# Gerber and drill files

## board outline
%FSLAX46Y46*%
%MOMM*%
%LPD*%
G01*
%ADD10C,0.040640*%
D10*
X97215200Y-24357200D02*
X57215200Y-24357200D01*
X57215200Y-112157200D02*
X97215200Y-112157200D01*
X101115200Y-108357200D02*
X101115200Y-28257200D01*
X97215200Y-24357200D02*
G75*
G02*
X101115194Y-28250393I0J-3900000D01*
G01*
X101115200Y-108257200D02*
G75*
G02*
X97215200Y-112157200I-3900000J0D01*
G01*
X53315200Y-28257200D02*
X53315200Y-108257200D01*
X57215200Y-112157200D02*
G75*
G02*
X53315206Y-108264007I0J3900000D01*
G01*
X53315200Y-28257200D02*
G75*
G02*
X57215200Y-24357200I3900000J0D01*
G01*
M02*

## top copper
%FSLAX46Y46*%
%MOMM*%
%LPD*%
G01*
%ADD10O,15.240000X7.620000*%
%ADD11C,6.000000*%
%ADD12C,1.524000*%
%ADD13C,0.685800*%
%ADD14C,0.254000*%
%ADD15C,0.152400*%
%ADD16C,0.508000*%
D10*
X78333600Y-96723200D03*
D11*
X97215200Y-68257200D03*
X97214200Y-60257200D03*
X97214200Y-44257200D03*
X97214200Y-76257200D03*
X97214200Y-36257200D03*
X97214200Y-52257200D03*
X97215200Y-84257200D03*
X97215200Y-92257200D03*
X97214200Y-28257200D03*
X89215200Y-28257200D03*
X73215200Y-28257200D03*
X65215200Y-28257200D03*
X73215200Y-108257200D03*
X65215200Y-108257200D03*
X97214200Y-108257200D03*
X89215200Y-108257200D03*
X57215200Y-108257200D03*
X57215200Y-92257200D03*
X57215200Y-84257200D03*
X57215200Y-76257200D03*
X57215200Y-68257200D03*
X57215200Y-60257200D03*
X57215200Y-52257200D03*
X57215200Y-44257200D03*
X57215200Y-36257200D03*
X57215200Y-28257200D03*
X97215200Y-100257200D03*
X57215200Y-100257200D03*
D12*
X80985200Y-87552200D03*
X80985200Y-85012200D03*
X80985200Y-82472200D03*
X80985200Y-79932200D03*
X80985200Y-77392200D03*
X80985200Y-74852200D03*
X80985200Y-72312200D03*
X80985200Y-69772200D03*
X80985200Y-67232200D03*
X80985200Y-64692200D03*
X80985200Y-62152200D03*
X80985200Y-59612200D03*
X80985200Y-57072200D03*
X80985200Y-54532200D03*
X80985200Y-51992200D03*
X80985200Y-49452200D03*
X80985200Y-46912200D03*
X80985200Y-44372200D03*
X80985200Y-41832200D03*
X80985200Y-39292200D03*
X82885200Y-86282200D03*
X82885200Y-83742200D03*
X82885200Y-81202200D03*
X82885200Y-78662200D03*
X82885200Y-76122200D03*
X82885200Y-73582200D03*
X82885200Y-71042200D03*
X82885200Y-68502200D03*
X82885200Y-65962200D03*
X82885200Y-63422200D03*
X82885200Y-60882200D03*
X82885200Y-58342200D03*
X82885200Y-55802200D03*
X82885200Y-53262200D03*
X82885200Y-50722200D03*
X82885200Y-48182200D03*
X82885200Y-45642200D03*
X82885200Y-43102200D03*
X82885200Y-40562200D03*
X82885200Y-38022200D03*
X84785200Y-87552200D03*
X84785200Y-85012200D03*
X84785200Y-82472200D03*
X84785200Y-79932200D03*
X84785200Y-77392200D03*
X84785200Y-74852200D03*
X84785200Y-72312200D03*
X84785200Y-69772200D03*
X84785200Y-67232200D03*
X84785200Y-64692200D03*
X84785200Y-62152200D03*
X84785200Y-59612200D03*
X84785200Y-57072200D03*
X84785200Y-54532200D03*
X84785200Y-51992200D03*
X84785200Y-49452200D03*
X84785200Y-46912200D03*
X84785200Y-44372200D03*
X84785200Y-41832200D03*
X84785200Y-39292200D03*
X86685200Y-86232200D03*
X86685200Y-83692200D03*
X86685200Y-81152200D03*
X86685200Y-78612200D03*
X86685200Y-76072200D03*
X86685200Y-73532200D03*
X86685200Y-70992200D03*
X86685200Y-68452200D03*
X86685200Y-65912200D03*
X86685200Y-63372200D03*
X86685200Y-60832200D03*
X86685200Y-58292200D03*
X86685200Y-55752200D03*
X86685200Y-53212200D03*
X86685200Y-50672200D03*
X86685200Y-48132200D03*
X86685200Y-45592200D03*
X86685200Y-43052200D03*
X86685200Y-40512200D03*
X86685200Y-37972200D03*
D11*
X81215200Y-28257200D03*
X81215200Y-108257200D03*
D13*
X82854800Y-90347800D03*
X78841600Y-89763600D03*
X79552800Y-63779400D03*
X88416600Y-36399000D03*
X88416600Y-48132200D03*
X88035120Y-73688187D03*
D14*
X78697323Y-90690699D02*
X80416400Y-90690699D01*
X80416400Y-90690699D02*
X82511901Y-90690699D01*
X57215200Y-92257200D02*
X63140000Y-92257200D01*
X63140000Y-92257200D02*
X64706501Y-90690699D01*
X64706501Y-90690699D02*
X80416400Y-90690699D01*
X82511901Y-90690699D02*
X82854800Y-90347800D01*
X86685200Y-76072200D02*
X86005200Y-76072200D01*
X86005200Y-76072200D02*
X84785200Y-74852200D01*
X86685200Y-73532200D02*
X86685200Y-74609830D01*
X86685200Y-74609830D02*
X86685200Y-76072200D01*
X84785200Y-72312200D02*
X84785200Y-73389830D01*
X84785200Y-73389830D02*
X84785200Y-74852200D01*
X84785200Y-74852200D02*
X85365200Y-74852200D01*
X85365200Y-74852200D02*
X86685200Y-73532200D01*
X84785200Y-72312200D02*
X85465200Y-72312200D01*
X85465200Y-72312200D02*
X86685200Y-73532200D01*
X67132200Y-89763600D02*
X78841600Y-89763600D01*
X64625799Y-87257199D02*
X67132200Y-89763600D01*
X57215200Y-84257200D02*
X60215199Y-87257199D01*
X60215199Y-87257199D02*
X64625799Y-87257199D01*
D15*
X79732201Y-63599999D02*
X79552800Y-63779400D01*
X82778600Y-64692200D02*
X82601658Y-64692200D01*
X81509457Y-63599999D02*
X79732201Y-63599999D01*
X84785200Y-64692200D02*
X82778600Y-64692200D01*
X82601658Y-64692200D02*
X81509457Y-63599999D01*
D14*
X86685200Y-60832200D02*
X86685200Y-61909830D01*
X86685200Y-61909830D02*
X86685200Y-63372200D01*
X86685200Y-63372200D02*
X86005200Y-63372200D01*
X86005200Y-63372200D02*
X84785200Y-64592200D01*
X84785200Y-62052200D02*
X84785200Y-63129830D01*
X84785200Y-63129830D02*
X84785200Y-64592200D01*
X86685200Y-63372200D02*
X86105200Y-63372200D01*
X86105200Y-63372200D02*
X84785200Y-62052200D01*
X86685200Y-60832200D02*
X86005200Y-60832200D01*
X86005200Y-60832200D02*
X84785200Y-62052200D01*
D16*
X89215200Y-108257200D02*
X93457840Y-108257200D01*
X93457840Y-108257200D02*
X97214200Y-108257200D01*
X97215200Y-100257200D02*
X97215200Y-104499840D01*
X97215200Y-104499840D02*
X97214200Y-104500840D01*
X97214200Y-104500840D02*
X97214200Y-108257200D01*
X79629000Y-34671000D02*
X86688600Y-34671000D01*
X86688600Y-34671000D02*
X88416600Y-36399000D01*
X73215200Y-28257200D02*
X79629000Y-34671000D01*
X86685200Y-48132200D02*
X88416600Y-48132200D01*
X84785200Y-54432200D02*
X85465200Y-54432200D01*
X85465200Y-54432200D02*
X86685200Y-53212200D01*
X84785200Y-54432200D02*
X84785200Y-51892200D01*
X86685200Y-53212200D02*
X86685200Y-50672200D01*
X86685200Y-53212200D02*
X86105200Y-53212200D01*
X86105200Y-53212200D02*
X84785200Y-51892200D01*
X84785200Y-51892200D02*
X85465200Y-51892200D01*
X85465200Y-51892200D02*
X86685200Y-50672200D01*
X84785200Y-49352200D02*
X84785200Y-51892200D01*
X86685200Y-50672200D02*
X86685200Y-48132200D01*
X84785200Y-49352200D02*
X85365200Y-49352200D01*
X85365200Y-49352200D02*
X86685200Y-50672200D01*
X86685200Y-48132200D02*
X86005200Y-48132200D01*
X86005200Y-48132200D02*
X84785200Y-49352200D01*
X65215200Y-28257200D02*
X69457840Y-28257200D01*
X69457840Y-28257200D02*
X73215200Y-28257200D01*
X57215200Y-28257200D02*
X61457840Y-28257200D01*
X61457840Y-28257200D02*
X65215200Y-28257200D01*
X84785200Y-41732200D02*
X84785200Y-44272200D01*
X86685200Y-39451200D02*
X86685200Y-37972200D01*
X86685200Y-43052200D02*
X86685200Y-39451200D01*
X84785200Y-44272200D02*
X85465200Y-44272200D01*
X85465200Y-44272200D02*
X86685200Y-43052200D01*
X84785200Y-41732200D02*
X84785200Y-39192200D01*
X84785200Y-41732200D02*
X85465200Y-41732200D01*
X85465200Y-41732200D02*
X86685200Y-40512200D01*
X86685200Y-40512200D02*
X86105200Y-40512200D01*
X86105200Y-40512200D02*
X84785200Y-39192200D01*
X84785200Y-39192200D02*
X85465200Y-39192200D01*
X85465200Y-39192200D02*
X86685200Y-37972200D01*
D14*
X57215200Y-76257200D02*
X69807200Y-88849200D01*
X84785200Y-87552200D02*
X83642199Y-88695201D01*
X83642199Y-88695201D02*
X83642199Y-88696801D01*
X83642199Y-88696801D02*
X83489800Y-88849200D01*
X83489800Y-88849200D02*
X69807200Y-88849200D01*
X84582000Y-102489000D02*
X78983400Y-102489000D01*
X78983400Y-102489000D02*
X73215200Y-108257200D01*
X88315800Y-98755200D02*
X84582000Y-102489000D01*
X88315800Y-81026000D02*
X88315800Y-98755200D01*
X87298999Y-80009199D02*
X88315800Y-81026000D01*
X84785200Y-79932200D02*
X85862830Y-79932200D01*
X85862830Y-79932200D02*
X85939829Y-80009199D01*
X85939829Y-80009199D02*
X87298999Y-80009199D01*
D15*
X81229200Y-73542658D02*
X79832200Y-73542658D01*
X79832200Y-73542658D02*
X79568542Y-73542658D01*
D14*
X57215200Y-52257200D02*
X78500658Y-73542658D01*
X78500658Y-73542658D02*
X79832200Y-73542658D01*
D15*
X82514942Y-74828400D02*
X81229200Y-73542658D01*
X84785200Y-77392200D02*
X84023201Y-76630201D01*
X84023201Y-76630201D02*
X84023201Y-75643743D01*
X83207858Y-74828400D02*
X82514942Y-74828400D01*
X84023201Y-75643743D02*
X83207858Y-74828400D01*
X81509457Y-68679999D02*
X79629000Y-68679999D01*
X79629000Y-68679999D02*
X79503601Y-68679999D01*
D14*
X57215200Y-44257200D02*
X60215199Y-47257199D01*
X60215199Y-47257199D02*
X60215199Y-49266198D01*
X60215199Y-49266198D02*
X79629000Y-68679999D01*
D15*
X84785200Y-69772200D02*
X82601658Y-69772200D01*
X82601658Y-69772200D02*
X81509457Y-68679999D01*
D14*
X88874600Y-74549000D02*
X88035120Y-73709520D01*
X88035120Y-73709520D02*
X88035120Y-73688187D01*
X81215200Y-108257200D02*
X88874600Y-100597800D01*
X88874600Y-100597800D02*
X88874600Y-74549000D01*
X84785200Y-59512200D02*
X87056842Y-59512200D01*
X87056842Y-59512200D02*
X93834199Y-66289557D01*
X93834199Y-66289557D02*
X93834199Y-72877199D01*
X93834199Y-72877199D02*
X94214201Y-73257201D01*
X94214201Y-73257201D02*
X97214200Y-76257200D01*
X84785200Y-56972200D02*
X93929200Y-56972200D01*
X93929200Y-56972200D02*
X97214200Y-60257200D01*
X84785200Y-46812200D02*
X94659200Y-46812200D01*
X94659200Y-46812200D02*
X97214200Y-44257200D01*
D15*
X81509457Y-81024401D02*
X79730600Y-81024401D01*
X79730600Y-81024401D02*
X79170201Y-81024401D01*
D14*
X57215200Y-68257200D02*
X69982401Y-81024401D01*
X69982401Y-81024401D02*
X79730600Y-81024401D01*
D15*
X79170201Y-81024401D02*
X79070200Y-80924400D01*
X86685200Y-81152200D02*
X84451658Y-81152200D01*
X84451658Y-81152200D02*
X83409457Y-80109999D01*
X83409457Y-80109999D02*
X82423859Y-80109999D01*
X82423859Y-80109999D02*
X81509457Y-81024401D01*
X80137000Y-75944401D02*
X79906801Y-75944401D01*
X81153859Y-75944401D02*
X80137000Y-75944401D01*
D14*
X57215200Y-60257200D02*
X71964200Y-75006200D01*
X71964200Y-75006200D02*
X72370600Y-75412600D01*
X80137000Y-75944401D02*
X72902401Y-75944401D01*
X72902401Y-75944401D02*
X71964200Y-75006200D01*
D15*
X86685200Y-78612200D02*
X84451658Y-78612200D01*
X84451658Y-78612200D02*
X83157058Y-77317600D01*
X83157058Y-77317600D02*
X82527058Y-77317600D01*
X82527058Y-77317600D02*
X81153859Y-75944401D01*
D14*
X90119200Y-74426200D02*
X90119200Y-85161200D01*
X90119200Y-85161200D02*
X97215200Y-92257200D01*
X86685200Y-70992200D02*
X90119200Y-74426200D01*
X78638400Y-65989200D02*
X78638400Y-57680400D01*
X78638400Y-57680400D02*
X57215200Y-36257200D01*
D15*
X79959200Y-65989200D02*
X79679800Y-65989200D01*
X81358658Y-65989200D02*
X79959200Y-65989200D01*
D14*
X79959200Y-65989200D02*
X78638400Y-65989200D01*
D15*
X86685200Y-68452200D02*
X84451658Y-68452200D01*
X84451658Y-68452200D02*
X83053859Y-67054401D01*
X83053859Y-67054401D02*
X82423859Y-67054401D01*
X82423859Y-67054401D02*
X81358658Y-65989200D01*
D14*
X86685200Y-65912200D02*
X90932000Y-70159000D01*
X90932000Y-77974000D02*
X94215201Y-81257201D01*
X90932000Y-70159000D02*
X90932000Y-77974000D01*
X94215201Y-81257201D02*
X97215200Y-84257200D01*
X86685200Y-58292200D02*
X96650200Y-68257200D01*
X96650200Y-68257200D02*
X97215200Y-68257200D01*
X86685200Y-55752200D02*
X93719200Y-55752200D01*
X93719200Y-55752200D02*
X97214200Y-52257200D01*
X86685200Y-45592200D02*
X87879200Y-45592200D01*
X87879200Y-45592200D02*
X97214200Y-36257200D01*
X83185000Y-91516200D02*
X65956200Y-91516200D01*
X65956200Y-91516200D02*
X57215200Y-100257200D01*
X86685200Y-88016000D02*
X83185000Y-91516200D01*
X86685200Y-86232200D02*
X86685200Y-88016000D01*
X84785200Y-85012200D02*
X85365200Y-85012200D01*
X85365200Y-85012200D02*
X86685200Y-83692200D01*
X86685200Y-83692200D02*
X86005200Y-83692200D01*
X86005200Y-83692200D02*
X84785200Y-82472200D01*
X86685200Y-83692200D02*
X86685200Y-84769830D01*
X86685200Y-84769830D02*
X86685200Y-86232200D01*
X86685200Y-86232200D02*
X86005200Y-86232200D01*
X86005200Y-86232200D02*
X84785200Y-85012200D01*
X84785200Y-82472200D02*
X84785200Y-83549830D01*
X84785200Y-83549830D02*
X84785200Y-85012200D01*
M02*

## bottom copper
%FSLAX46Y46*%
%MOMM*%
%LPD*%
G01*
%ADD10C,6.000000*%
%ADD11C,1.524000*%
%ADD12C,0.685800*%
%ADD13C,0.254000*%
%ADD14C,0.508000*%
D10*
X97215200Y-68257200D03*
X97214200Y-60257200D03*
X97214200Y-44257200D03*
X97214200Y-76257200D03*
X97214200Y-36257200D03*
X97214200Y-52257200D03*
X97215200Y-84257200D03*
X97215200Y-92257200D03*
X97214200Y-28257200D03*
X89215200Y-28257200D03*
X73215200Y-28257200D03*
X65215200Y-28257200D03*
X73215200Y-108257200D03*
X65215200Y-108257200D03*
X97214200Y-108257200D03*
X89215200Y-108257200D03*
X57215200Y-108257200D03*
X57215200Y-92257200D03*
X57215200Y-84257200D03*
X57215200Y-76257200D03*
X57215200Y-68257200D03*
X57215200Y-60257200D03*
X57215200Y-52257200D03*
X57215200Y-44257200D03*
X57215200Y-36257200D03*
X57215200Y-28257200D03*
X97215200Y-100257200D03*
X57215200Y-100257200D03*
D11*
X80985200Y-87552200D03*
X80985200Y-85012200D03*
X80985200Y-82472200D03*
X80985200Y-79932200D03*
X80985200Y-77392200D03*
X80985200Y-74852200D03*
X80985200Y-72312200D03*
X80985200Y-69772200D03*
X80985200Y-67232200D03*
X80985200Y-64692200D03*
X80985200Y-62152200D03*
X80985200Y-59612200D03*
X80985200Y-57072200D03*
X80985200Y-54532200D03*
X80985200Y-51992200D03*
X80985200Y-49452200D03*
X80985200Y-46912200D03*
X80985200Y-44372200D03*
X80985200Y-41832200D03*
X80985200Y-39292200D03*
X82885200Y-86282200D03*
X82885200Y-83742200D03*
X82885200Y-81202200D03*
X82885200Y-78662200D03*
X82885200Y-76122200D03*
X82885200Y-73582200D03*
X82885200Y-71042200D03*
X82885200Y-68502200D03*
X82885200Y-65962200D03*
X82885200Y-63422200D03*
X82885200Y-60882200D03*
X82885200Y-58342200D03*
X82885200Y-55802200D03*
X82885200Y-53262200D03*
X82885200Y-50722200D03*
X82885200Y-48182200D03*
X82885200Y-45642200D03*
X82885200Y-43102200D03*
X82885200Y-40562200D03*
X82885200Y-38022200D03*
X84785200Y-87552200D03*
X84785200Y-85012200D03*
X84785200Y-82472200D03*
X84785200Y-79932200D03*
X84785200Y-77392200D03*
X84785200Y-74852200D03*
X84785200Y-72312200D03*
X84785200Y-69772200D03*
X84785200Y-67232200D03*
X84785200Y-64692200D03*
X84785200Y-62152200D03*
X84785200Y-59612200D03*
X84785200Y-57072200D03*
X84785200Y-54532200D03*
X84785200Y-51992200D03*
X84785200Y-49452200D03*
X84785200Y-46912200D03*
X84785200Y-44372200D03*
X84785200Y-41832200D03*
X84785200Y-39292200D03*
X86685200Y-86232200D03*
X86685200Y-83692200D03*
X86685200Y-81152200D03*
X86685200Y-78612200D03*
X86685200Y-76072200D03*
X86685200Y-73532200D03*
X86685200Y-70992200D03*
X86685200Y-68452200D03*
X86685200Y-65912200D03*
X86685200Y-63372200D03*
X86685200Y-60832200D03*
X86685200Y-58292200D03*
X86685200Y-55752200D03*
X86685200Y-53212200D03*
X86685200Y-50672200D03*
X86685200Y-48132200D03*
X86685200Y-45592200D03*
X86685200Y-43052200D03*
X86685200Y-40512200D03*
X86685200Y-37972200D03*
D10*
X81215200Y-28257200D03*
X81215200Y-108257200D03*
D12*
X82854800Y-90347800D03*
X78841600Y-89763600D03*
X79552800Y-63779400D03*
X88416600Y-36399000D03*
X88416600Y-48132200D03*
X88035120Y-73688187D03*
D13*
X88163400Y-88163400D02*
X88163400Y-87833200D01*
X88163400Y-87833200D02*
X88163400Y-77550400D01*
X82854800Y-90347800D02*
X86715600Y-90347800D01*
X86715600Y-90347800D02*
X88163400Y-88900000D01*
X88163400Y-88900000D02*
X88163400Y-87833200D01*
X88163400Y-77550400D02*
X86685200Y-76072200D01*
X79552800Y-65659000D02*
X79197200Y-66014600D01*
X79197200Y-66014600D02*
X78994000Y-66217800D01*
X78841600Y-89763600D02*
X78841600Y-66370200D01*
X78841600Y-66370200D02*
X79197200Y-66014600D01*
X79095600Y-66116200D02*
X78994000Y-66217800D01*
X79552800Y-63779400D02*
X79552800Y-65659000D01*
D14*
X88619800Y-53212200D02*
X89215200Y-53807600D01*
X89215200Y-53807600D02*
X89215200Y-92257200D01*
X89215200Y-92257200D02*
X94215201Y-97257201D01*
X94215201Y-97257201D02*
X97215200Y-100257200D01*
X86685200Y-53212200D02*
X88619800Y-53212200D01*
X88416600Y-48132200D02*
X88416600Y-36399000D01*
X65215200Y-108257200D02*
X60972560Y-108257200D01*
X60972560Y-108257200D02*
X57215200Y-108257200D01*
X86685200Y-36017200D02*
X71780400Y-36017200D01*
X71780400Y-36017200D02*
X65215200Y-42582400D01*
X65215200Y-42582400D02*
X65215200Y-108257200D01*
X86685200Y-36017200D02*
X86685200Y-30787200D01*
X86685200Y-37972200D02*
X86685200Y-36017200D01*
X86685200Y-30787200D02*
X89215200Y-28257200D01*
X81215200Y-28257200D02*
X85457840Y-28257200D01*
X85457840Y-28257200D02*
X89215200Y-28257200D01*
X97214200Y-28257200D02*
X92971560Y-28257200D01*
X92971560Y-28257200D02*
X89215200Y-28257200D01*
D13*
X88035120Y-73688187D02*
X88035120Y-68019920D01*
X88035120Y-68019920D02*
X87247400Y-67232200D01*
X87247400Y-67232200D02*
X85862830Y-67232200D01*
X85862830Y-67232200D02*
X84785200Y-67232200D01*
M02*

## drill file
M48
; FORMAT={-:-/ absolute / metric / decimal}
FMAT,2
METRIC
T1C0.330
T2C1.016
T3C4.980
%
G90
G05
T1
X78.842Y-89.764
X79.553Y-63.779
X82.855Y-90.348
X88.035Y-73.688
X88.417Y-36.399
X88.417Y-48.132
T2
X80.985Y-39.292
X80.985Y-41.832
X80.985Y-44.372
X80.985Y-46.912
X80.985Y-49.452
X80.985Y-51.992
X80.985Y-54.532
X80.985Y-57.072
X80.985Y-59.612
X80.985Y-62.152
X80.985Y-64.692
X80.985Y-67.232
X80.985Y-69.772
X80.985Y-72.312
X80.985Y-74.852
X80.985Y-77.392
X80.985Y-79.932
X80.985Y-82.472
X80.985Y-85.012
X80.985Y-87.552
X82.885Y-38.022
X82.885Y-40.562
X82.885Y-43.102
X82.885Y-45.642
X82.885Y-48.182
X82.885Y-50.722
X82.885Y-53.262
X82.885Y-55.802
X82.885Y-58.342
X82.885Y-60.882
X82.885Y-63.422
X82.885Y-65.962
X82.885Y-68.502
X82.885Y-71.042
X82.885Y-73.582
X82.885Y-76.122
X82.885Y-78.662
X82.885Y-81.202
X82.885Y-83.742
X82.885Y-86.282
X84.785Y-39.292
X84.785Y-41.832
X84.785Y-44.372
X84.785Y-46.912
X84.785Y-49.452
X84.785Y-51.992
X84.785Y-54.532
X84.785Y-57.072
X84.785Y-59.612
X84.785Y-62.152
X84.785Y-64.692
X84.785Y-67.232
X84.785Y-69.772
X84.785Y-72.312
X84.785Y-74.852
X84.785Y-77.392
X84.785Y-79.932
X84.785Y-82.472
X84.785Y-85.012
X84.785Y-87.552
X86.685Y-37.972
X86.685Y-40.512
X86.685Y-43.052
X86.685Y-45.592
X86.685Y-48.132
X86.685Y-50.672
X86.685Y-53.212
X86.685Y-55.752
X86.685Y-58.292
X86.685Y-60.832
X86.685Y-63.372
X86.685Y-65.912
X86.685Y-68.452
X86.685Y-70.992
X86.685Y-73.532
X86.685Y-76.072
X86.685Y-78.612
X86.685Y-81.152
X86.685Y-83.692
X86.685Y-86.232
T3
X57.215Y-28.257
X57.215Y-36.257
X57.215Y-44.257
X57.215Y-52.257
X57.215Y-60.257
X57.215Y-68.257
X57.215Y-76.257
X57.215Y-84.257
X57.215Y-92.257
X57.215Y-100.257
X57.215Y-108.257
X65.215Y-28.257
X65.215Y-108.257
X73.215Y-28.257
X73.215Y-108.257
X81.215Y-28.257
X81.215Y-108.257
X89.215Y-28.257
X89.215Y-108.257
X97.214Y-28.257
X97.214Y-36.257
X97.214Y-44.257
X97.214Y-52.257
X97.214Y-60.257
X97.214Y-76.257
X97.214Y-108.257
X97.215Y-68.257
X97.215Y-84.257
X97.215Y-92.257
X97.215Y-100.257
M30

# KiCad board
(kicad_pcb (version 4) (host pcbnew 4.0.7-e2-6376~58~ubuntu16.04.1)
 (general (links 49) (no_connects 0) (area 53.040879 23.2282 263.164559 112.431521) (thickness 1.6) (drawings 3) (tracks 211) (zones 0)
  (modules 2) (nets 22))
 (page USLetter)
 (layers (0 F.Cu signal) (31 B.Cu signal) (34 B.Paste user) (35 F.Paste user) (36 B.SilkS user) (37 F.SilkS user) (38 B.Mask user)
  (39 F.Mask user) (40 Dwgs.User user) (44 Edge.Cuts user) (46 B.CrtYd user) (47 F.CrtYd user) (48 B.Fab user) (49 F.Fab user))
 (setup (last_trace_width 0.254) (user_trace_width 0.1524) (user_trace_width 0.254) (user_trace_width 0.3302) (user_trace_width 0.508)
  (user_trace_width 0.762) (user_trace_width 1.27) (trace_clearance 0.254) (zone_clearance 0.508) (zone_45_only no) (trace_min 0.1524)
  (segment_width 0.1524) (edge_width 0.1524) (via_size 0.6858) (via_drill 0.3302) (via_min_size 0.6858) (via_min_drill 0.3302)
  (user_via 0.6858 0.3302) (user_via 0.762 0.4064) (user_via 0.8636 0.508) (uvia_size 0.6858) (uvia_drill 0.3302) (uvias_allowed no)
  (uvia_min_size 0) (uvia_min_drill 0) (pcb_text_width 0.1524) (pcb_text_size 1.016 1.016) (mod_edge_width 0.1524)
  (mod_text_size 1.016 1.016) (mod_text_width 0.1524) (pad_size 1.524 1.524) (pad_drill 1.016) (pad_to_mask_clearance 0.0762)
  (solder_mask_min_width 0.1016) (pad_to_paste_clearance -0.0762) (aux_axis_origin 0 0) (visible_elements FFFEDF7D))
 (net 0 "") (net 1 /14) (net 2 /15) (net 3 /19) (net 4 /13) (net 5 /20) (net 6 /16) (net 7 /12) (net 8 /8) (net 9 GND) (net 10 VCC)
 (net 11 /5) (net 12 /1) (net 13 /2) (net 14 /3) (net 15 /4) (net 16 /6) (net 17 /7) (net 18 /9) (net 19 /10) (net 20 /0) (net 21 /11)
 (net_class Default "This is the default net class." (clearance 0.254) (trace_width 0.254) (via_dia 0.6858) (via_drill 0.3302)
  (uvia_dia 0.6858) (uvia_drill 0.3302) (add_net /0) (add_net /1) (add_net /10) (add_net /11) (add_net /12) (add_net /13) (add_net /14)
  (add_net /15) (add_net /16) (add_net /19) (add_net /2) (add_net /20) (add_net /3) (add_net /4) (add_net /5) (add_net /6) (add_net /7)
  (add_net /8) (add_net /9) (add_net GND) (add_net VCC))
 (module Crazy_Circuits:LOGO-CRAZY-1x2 (layer F.Cu) (at 78.3336 100.6602)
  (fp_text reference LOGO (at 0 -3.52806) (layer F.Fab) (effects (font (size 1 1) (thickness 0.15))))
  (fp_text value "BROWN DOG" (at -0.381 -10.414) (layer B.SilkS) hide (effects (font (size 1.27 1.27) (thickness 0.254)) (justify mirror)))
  (pad BG smd oval (at 0 -3.937) (size 15.24 7.62) (layers F.Cu)))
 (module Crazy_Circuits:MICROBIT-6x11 (layer F.Cu) (at 57.2152 28.2572)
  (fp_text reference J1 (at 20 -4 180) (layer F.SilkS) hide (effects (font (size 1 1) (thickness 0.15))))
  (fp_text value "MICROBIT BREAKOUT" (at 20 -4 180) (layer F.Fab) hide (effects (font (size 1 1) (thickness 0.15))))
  (fp_line (start 40 -3.9) (end 0 -3.9) (layer Edge.Cuts) (width 0.04064))
  (fp_line (start 0 83.9) (end 40 83.9) (layer Edge.Cuts) (width 0.04064))
  (fp_line (start 43.9 80.1) (end 43.9 0) (layer Edge.Cuts) (width 0.04064))
  (fp_arc (start 40 0) (end 40 -3.9) (angle 89.9) (layer Edge.Cuts) (width 0.04064))
  (fp_arc (start 40 80) (end 43.9 80) (angle 90) (layer Edge.Cuts) (width 0.04064))
  (fp_line (start -3.9 0) (end -3.9 80) (layer Edge.Cuts) (width 0.04064))
  (fp_arc (start 0 80) (end 0 83.9) (angle 89.9) (layer Edge.Cuts) (width 0.04064))
  (fp_arc (start 0 0) (end -3.9 0) (angle 90) (layer Edge.Cuts) (width 0.04064))
  (pad 14 thru_hole circle (at 40 40 270) (size 6 6) (drill 4.98) (layers *.Cu *.Mask) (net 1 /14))
  (pad 15 thru_hole circle (at 39.999 32 270) (size 6 6) (drill 4.98) (layers *.Cu *.Mask) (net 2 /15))
  (pad 19 thru_hole circle (at 39.999 16 270) (size 6 6) (drill 4.98) (layers *.Cu *.Mask) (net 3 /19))
  (pad 13 thru_hole circle (at 39.999 48 270) (size 6 6) (drill 4.98) (layers *.Cu *.Mask) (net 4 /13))
  (pad 20 thru_hole circle (at 39.999 8 270) (size 6 6) (drill 4.98) (layers *.Cu *.Mask) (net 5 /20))
  (pad 16 thru_hole circle (at 39.999 24 270) (size 6 6) (drill 4.98) (layers *.Cu *.Mask) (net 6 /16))
  (pad 12 thru_hole circle (at 40 56 270) (size 6 6) (drill 4.98) (layers *.Cu *.Mask) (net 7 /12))
  (pad 8 thru_hole circle (at 40 64 270) (size 6 6) (drill 4.98) (layers *.Cu *.Mask) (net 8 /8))
  (pad GND thru_hole circle (at 39.999 0 270) (size 6 6) (drill 4.98) (layers *.Cu *.Mask) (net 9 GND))
  (pad GND thru_hole circle (at 32 0 270) (size 6 6) (drill 4.98) (layers *.Cu *.Mask) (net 9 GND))
  (pad 3V thru_hole circle (at 16 0 270) (size 6 6) (drill 4.98) (layers *.Cu *.Mask) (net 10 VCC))
  (pad 3V thru_hole circle (at 8 0 270) (size 6 6) (drill 4.98) (layers *.Cu *.Mask) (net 10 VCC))
  (pad 5 thru_hole circle (at 16 80 270) (size 6 6) (drill 4.98) (layers *.Cu *.Mask) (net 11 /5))
  (pad GND thru_hole circle (at 8 80 270) (size 6 6) (drill 4.98) (layers *.Cu *.Mask) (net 9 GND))
  (pad 3V thru_hole circle (at 39.999 80 270) (size 6 6) (drill 4.98) (layers *.Cu *.Mask) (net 10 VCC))
  (pad 3V thru_hole circle (at 32 80 270) (size 6 6) (drill 4.98) (layers *.Cu *.Mask) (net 10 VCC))
  (pad GND thru_hole circle (at 0 80 270) (size 6 6) (drill 4.98) (layers *.Cu *.Mask) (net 9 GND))
  (pad 1 thru_hole circle (at 0 64 270) (size 6 6) (drill 4.98) (layers *.Cu *.Mask) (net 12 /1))
  (pad 2 thru_hole circle (at 0 56 270) (size 6 6) (drill 4.98) (layers *.Cu *.Mask) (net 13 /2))
  (pad 3 thru_hole circle (at 0 48 270) (size 6 6) (drill 4.98) (layers *.Cu *.Mask) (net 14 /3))
  (pad 4 thru_hole circle (at 0 40 270) (size 6 6) (drill 4.98) (layers *.Cu *.Mask) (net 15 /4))
  (pad 6 thru_hole circle (at 0 32 270) (size 6 6) (drill 4.98) (layers *.Cu *.Mask) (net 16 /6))
  (pad 7 thru_hole circle (at 0 24 270) (size 6 6) (drill 4.98) (layers *.Cu *.Mask) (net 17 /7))
  (pad 9 thru_hole circle (at 0 16 270) (size 6 6) (drill 4.98) (layers *.Cu *.Mask) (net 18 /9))
  (pad 10 thru_hole circle (at 0 8 270) (size 6 6) (drill 4.98) (layers *.Cu *.Mask) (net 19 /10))
  (pad 3V thru_hole circle (at 0 0 270) (size 6 6) (drill 4.98) (layers *.Cu *.Mask) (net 10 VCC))
  (pad 3V thru_hole circle (at 40 72 270) (size 6 6) (drill 4.98) (layers *.Cu *.Mask) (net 10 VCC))
  (pad 0 thru_hole circle (at 0 72 270) (size 6 6) (drill 4.98) (layers *.Cu *.Mask) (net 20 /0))
  (pad NC thru_hole circle (at 23.77 59.295 90) (size 1.524 1.524) (drill 1.016) (layers *.Cu *.Mask F.SilkS))
  (pad NC thru_hole circle (at 23.77 56.755 90) (size 1.524 1.524) (drill 1.016) (layers *.Cu *.Mask F.SilkS))
  (pad NC thru_hole circle (at 23.77 54.215 90) (size 1.524 1.524) (drill 1.016) (layers *.Cu *.Mask F.SilkS))
  (pad NC thru_hole circle (at 23.77 51.675 90) (size 1.524 1.524) (drill 1.016) (layers *.Cu *.Mask F.SilkS))
  (pad NC thru_hole circle (at 23.77 49.135 90) (size 1.524 1.524) (drill 1.016) (layers *.Cu *.Mask F.SilkS))
  (pad NC thru_hole circle (at 23.77 46.595 90) (size 1.524 1.524) (drill 1.016) (layers *.Cu *.Mask F.SilkS))
  (pad NC thru_hole circle (at 23.77 44.055 90) (size 1.524 1.524) (drill 1.016) (layers *.Cu *.Mask F.SilkS))
  (pad NC thru_hole circle (at 23.77 41.515 90) (size 1.524 1.524) (drill 1.016) (layers *.Cu *.Mask F.SilkS))
  (pad NC thru_hole circle (at 23.77 38.975 90) (size 1.524 1.524) (drill 1.016) (layers *.Cu *.Mask F.SilkS))
  (pad NC thru_hole circle (at 23.77 36.435 90) (size 1.524 1.524) (drill 1.016) (layers *.Cu *.Mask F.SilkS))
  (pad NC thru_hole circle (at 23.77 33.895 90) (size 1.524 1.524) (drill 1.016) (layers *.Cu *.Mask F.SilkS))
  (pad NC thru_hole circle (at 23.77 31.355 90) (size 1.524 1.524) (drill 1.016) (layers *.Cu *.Mask F.SilkS))
  (pad NC thru_hole circle (at 23.77 28.815 90) (size 1.524 1.524) (drill 1.016) (layers *.Cu *.Mask F.SilkS))
  (pad NC thru_hole circle (at 23.77 26.275 90) (size 1.524 1.524) (drill 1.016) (layers *.Cu *.Mask F.SilkS))
  (pad NC thru_hole circle (at 23.77 23.735 90) (size 1.524 1.524) (drill 1.016) (layers *.Cu *.Mask F.SilkS))
  (pad NC thru_hole circle (at 23.77 21.195 90) (size 1.524 1.524) (drill 1.016) (layers *.Cu *.Mask F.SilkS))
  (pad NC thru_hole circle (at 23.77 18.655 90) (size 1.524 1.524) (drill 1.016) (layers *.Cu *.Mask F.SilkS))
  (pad NC thru_hole circle (at 23.77 16.115 90) (size 1.524 1.524) (drill 1.016) (layers *.Cu *.Mask F.SilkS))
  (pad NC thru_hole circle (at 23.77 13.575 90) (size 1.524 1.524) (drill 1.016) (layers *.Cu *.Mask F.SilkS))
  (pad NC thru_hole circle (at 23.77 11.035 90) (size 1.524 1.524) (drill 1.016) (layers *.Cu *.Mask F.SilkS))
  (pad NC thru_hole circle (at 25.67 58.025 90) (size 1.524 1.524) (drill 1.016) (layers *.Cu *.Mask F.SilkS))
  (pad NC thru_hole circle (at 25.67 55.485 90) (size 1.524 1.524) (drill 1.016) (layers *.Cu *.Mask F.SilkS))
  (pad NC thru_hole circle (at 25.67 52.945 90) (size 1.524 1.524) (drill 1.016) (layers *.Cu *.Mask F.SilkS))
  (pad NC thru_hole circle (at 25.67 50.405 90) (size 1.524 1.524) (drill 1.016) (layers *.Cu *.Mask F.SilkS))
  (pad NC thru_hole circle (at 25.67 47.865 90) (size 1.524 1.524) (drill 1.016) (layers *.Cu *.Mask F.SilkS))
  (pad NC thru_hole circle (at 25.67 45.325 90) (size 1.524 1.524) (drill 1.016) (layers *.Cu *.Mask F.SilkS))
  (pad NC thru_hole circle (at 25.67 42.785 90) (size 1.524 1.524) (drill 1.016) (layers *.Cu *.Mask F.SilkS))
  (pad Nc thru_hole circle (at 25.67 40.245 90) (size 1.524 1.524) (drill 1.016) (layers *.Cu *.Mask F.SilkS))
  (pad NC thru_hole circle (at 25.67 37.705 90) (size 1.524 1.524) (drill 1.016) (layers *.Cu *.Mask F.SilkS))
  (pad NC thru_hole circle (at 25.67 35.165 90) (size 1.524 1.524) (drill 1.016) (layers *.Cu *.Mask F.SilkS))
  (pad NC thru_hole circle (at 25.67 32.625 90) (size 1.524 1.524) (drill 1.016) (layers *.Cu *.Mask F.SilkS))
  (pad NC thru_hole circle (at 25.67 30.085 90) (size 1.524 1.524) (drill 1.016) (layers *.Cu *.Mask F.SilkS))
  (pad NC thru_hole circle (at 25.67 27.545 90) (size 1.524 1.524) (drill 1.016) (layers *.Cu *.Mask F.SilkS))
  (pad NC thru_hole circle (at 25.67 25.005 90) (size 1.524 1.524) (drill 1.016) (layers *.Cu *.Mask F.SilkS))
  (pad NC thru_hole circle (at 25.67 22.465 90) (size 1.524 1.524) (drill 1.016) (layers *.Cu *.Mask F.SilkS))
  (pad NC thru_hole circle (at 25.67 19.925 90) (size 1.524 1.524) (drill 1.016) (layers *.Cu *.Mask F.SilkS))
  (pad NC thru_hole circle (at 25.67 17.385 90) (size 1.524 1.524) (drill 1.016) (layers *.Cu *.Mask F.SilkS))
  (pad NC thru_hole circle (at 25.67 14.845 90) (size 1.524 1.524) (drill 1.016) (layers *.Cu *.Mask F.SilkS))
  (pad NC thru_hole circle (at 25.67 12.305 90) (size 1.524 1.524) (drill 1.016) (layers *.Cu *.Mask F.SilkS))
  (pad NC thru_hole circle (at 25.67 9.765 90) (size 1.524 1.524) (drill 1.016) (layers *.Cu *.Mask F.SilkS))
  (pad 3 thru_hole circle (at 27.57 59.295 90) (size 1.524 1.524) (drill 1.016) (layers *.Cu *.Mask F.SilkS) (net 14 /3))
  (pad 0 thru_hole circle (at 27.57 56.755 90) (size 1.524 1.524) (drill 1.016) (layers *.Cu *.Mask F.SilkS) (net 20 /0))
  (pad 0 thru_hole circle (at 27.57 54.215 90) (size 1.524 1.524) (drill 1.016) (layers *.Cu *.Mask F.SilkS) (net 20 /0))
  (pad 5 thru_hole circle (at 27.57 51.675 90) (size 1.524 1.524) (drill 1.016) (layers *.Cu *.Mask F.SilkS) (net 11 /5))
  (pad 7 thru_hole circle (at 27.57 49.135 90) (size 1.524 1.524) (drill 1.016) (layers *.Cu *.Mask F.SilkS) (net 17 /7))
  (pad 1 thru_hole circle (at 27.57 46.595 90) (size 1.524 1.524) (drill 1.016) (layers *.Cu *.Mask F.SilkS) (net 12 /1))
  (pad 1 thru_hole circle (at 27.57 44.055 90) (size 1.524 1.524) (drill 1.016) (layers *.Cu *.Mask F.SilkS) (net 12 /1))
  (pad 9 thru_hole circle (at 27.57 41.515 90) (size 1.524 1.524) (drill 1.016) (layers *.Cu *.Mask F.SilkS) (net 18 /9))
  (pad 11 thru_hole circle (at 27.57 38.975 90) (size 1.524 1.524) (drill 1.016) (layers *.Cu *.Mask F.SilkS) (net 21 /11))
  (pad 2 thru_hole circle (at 27.57 36.435 90) (size 1.524 1.524) (drill 1.016) (layers *.Cu *.Mask F.SilkS) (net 13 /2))
  (pad 2 thru_hole circle (at 27.57 33.895 90) (size 1.524 1.524) (drill 1.016) (layers *.Cu *.Mask F.SilkS) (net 13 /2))
  (pad 13 thru_hole circle (at 27.57 31.355 90) (size 1.524 1.524) (drill 1.016) (layers *.Cu *.Mask F.SilkS) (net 4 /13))
  (pad 15 thru_hole circle (at 27.57 28.815 90) (size 1.524 1.524) (drill 1.016) (layers *.Cu *.Mask F.SilkS) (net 2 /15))
  (pad 3V thru_hole circle (at 27.57 26.275 90) (size 1.524 1.524) (drill 1.016) (layers *.Cu *.Mask F.SilkS) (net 10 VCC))
  (pad 3V thru_hole circle (at 27.57 23.735 90) (size 1.524 1.524) (drill 1.016) (layers *.Cu *.Mask F.SilkS) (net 10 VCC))
  (pad 3V thru_hole circle (at 27.57 21.195 90) (size 1.524 1.524) (drill 1.016) (layers *.Cu *.Mask F.SilkS) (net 10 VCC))
  (pad 19 thru_hole circle (at 27.57 18.655 90) (size 1.524 1.524) (drill 1.016) (layers *.Cu *.Mask F.SilkS) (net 3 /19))
  (pad GND thru_hole circle (at 27.57 16.115 90) (size 1.524 1.524) (drill 1.016) (layers *.Cu *.Mask F.SilkS) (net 9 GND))
  (pad GND thru_hole circle (at 27.57 13.575 90) (size 1.524 1.524) (drill 1.016) (layers *.Cu *.Mask F.SilkS) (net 9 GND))
  (pad GND thru_hole circle (at 27.57 11.035 90) (size 1.524 1.524) (drill 1.016) (layers *.Cu *.Mask F.SilkS) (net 9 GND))
  (pad 0 thru_hole circle (at 29.47 57.975 90) (size 1.524 1.524) (drill 1.016) (layers *.Cu *.Mask F.SilkS) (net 20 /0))
  (pad 0 thru_hole circle (at 29.47 55.435 90) (size 1.524 1.524) (drill 1.016) (layers *.Cu *.Mask F.SilkS) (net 20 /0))
  (pad 4 thru_hole circle (at 29.47 52.895 90) (size 1.524 1.524) (drill 1.016) (layers *.Cu *.Mask F.SilkS) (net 15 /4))
  (pad 6 thru_hole circle (at 29.47 50.355 90) (size 1.524 1.524) (drill 1.016) (layers *.Cu *.Mask F.SilkS) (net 16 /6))
  (pad 1 thru_hole circle (at 29.47 47.815 90) (size 1.524 1.524) (drill 1.016) (layers *.Cu *.Mask F.SilkS) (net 12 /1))
  (pad 1 thru_hole circle (at 29.47 45.275 90) (size 1.524 1.524) (drill 1.016) (layers *.Cu *.Mask F.SilkS) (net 12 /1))
  (pad 8 thru_hole circle (at 29.47 42.735 90) (size 1.524 1.524) (drill 1.016) (layers *.Cu *.Mask F.SilkS) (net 8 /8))
  (pad 10 thru_hole circle (at 29.47 40.195 90) (size 1.524 1.524) (drill 1.016) (layers *.Cu *.Mask F.SilkS) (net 19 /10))
  (pad 12 thru_hole circle (at 29.47 37.655 90) (size 1.524 1.524) (drill 1.016) (layers *.Cu *.Mask F.SilkS) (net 7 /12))
  (pad 2 thru_hole circle (at 29.47 35.115 90) (size 1.524 1.524) (drill 1.016) (layers *.Cu *.Mask F.SilkS) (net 13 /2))
  (pad 2 thru_hole circle (at 29.47 32.575 90) (size 1.524 1.524) (drill 1.016) (layers *.Cu *.Mask F.SilkS) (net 13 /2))
  (pad 14 thru_hole circle (at 29.47 30.035 90) (size 1.524 1.524) (drill 1.016) (layers *.Cu *.Mask F.SilkS) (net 1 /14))
  (pad 16 thru_hole circle (at 29.47 27.495 90) (size 1.524 1.524) (drill 1.016) (layers *.Cu *.Mask F.SilkS) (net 6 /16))
  (pad 3V thru_hole circle (at 29.47 24.955 90) (size 1.524 1.524) (drill 1.016) (layers *.Cu *.Mask F.SilkS) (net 10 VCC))
  (pad 3V thru_hole circle (at 29.47 22.415 90) (size 1.524 1.524) (drill 1.016) (layers *.Cu *.Mask F.SilkS) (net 10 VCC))
  (pad 3V thru_hole circle (at 29.47 19.875 90) (size 1.524 1.524) (drill 1.016) (layers *.Cu *.Mask F.SilkS) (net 10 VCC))
  (pad 20 thru_hole circle (at 29.47 17.335 90) (size 1.524 1.524) (drill 1.016) (layers *.Cu *.Mask F.SilkS) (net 5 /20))
  (pad GND thru_hole circle (at 29.47 14.795 90) (size 1.524 1.524) (drill 1.016) (layers *.Cu *.Mask F.SilkS) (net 9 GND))
  (pad GND thru_hole circle (at 29.47 12.255 90) (size 1.524 1.524) (drill 1.016) (layers *.Cu *.Mask F.SilkS) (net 9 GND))
  (pad GND thru_hole circle (at 29.47 9.715 90) (size 1.524 1.524) (drill 1.016) (layers *.Cu *.Mask F.SilkS) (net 9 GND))
  (pad GND thru_hole circle (at 24 0 270) (size 6 6) (drill 4.98) (layers *.Cu *.Mask) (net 9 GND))
  (pad 11 thru_hole circle (at 24 80 270) (size 6 6) (drill 4.98) (layers *.Cu *.Mask) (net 21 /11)))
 (segment (start 78.697323 90.690699) (end 80.4164 90.690699) (width 0.254) (layer F.Cu) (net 12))
 (segment (start 80.4164 90.690699) (end 82.511901 90.690699) (width 0.254) (layer F.Cu) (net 12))
 (segment (start 57.2152 92.2572) (end 63.14 92.2572) (width 0.254) (layer F.Cu) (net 12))
 (segment (start 63.14 92.2572) (end 64.706501 90.690699) (width 0.254) (layer F.Cu) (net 12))
 (segment (start 64.706501 90.690699) (end 80.4164 90.690699) (width 0.254) (layer F.Cu) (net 12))
 (segment (start 82.511901 90.690699) (end 82.8548 90.3478) (width 0.254) (layer F.Cu) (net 12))
 (segment (start 88.1634 88.1634) (end 88.1634 87.8332) (width 0.254) (layer B.Cu) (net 12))
 (segment (start 88.1634 87.8332) (end 88.1634 77.5504) (width 0.254) (layer B.Cu) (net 12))
 (segment (start 82.8548 90.3478) (end 86.7156 90.3478) (width 0.254) (layer B.Cu) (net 12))
 (segment (start 86.7156 90.3478) (end 88.1634 88.9) (width 0.254) (layer B.Cu) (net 12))
 (segment (start 88.1634 88.9) (end 88.1634 87.8332) (width 0.254) (layer B.Cu) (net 12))
 (via (at 82.8548 90.3478) (size 0.6858) (drill 0.3302) (layers F.Cu B.Cu) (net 12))
 (segment (start 88.1634 77.5504) (end 86.6852 76.0722) (width 0.254) (layer B.Cu) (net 12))
 (segment (start 86.6852 76.0722) (end 86.0052 76.0722) (width 0.254) (layer F.Cu) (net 12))
 (segment (start 86.0052 76.0722) (end 84.7852 74.8522) (width 0.254) (layer F.Cu) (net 12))
 (segment (start 86.6852 73.5322) (end 86.6852 74.60983) (width 0.254) (layer F.Cu) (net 12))
 (segment (start 86.6852 74.60983) (end 86.6852 76.0722) (width 0.254) (layer F.Cu) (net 12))
 (segment (start 84.7852 72.3122) (end 84.7852 73.38983) (width 0.254) (layer F.Cu) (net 12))
 (segment (start 84.7852 73.38983) (end 84.7852 74.8522) (width 0.254) (layer F.Cu) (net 12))
 (segment (start 84.7852 74.8522) (end 85.3652 74.8522) (width 0.254) (layer F.Cu) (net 12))
 (segment (start 85.3652 74.8522) (end 86.6852 73.5322) (width 0.254) (layer F.Cu) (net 12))
 (segment (start 84.7852 72.3122) (end 85.4652 72.3122) (width 0.254) (layer F.Cu) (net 12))
 (segment (start 85.4652 72.3122) (end 86.6852 73.5322) (width 0.254) (layer F.Cu) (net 12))
 (segment (start 79.5528 65.659) (end 79.1972 66.0146) (width 0.254) (layer B.Cu) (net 13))
 (segment (start 79.1972 66.0146) (end 78.994 66.2178) (width 0.254) (layer B.Cu) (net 13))
 (segment (start 78.8416 89.7636) (end 78.8416 66.3702) (width 0.254) (layer B.Cu) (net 13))
 (segment (start 78.8416 66.3702) (end 79.1972 66.0146) (width 0.254) (layer B.Cu) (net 13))
 (segment (start 67.1322 89.7636) (end 78.8416 89.7636) (width 0.254) (layer F.Cu) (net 13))
 (via (at 78.8416 89.7636) (size 0.6858) (drill 0.3302) (layers F.Cu B.Cu) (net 13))
 (segment (start 64.625799 87.257199) (end 67.1322 89.7636) (width 0.254) (layer F.Cu) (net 13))
 (segment (start 57.2152 84.2572) (end 60.215199 87.257199) (width 0.254) (layer F.Cu) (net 13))
 (segment (start 60.215199 87.257199) (end 64.625799 87.257199) (width 0.254) (layer F.Cu) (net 13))
 (segment (start 79.0956 66.1162) (end 78.994 66.2178) (width 0.254) (layer B.Cu) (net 13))
 (segment (start 79.5528 63.7794) (end 79.5528 65.659) (width 0.254) (layer B.Cu) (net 13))
 (segment (start 79.732201 63.599999) (end 79.5528 63.7794) (width 0.1524) (layer F.Cu) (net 13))
 (via (at 79.5528 63.7794) (size 0.6858) (drill 0.3302) (layers F.Cu B.Cu) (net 13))
 (segment (start 82.7786 64.6922) (end 82.601658 64.6922) (width 0.1524) (layer F.Cu) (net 13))
 (segment (start 81.509457 63.599999) (end 79.732201 63.599999) (width 0.1524) (layer F.Cu) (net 13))
 (segment (start 84.7852 64.6922) (end 82.7786 64.6922) (width 0.1524) (layer F.Cu) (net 13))
 (segment (start 82.601658 64.6922) (end 81.509457 63.599999) (width 0.1524) (layer F.Cu) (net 13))
 (segment (start 86.6852 60.8322) (end 86.6852 61.90983) (width 0.254) (layer F.Cu) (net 13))
 (segment (start 86.6852 61.90983) (end 86.6852 63.3722) (width 0.254) (layer F.Cu) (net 13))
 (segment (start 86.6852 63.3722) (end 86.0052 63.3722) (width 0.254) (layer F.Cu) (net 13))
 (segment (start 86.0052 63.3722) (end 84.7852 64.5922) (width 0.254) (layer F.Cu) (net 13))
 (segment (start 84.7852 62.0522) (end 84.7852 63.12983) (width 0.254) (layer F.Cu) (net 13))
 (segment (start 84.7852 63.12983) (end 84.7852 64.5922) (width 0.254) (layer F.Cu) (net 13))
 (segment (start 86.6852 63.3722) (end 86.1052 63.3722) (width 0.254) (layer F.Cu) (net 13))
 (segment (start 86.1052 63.3722) (end 84.7852 62.0522) (width 0.254) (layer F.Cu) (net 13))
 (segment (start 86.6852 60.8322) (end 86.0052 60.8322) (width 0.254) (layer F.Cu) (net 13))
 (segment (start 86.0052 60.8322) (end 84.7852 62.0522) (width 0.254) (layer F.Cu) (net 13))
 (segment (start 89.2152 108.2572) (end 93.45784 108.2572) (width 0.508) (layer F.Cu) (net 10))
 (segment (start 93.45784 108.2572) (end 97.2142 108.2572) (width 0.508) (layer F.Cu) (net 10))
 (segment (start 97.2152 100.2572) (end 97.2152 104.49984) (width 0.508) (layer F.Cu) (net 10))
 (segment (start 97.2152 104.49984) (end 97.2142 104.50084) (width 0.508) (layer F.Cu) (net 10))
 (segment (start 97.2142 104.50084) (end 97.2142 108.2572) (width 0.508) (layer F.Cu) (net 10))
 (segment (start 79.629 34.671) (end 86.6886 34.671) (width 0.508) (layer F.Cu) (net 10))
 (segment (start 86.6886 34.671) (end 88.4166 36.399) (width 0.508) (layer F.Cu) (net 10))
 (segment (start 73.2152 28.2572) (end 79.629 34.671) (width 0.508) (layer F.Cu) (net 10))
 (segment (start 88.6198 53.2122) (end 89.2152 53.8076) (width 0.508) (layer B.Cu) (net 10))
 (segment (start 89.2152 53.8076) (end 89.2152 92.2572) (width 0.508) (layer B.Cu) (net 10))
 (segment (start 89.2152 92.2572) (end 94.215201 97.257201) (width 0.508) (layer B.Cu) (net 10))
 (segment (start 94.215201 97.257201) (end 97.2152 100.2572) (width 0.508) (layer B.Cu) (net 10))
 (segment (start 86.6852 53.2122) (end 88.6198 53.2122) (width 0.508) (layer B.Cu) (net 10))
 (via (at 88.4166 36.399) (size 0.6858) (drill 0.3302) (layers F.Cu B.Cu) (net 10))
 (segment (start 88.4166 48.1322) (end 88.4166 36.399) (width 0.508) (layer B.Cu) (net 10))
 (via (at 88.4166 48.1322) (size 0.6858) (drill 0.3302) (layers F.Cu B.Cu) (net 10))
 (segment (start 86.6852 48.1322) (end 88.4166 48.1322) (width 0.508) (layer F.Cu) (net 10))
 (segment (start 84.7852 54.4322) (end 85.4652 54.4322) (width 0.508) (layer F.Cu) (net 10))
 (segment (start 85.4652 54.4322) (end 86.6852 53.2122) (width 0.508) (layer F.Cu) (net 10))
 (segment (start 84.7852 54.4322) (end 84.7852 51.8922) (width 0.508) (layer F.Cu) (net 10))
 (segment (start 86.6852 53.2122) (end 86.6852 50.6722) (width 0.508) (layer F.Cu) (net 10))
 (segment (start 86.6852 53.2122) (end 86.1052 53.2122) (width 0.508) (layer F.Cu) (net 10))
 (segment (start 86.1052 53.2122) (end 84.7852 51.8922) (width 0.508) (layer F.Cu) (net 10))
 (segment (start 84.7852 51.8922) (end 85.4652 51.8922) (width 0.508) (layer F.Cu) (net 10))
 (segment (start 85.4652 51.8922) (end 86.6852 50.6722) (width 0.508) (layer F.Cu) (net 10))
 (segment (start 84.7852 49.3522) (end 84.7852 51.8922) (width 0.508) (layer F.Cu) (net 10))
 (segment (start 86.6852 50.6722) (end 86.6852 48.1322) (width 0.508) (layer F.Cu) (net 10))
 (segment (start 84.7852 49.3522) (end 85.3652 49.3522) (width 0.508) (layer F.Cu) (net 10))
 (segment (start 85.3652 49.3522) (end 86.6852 50.6722) (width 0.508) (layer F.Cu) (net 10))
 (segment (start 86.6852 48.1322) (end 86.0052 48.1322) (width 0.508) (layer F.Cu) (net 10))
 (segment (start 86.0052 48.1322) (end 84.7852 49.3522) (width 0.508) (layer F.Cu) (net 10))
 (segment (start 65.2152 28.2572) (end 69.45784 28.2572) (width 0.508) (layer F.Cu) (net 10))
 (segment (start 69.45784 28.2572) (end 73.2152 28.2572) (width 0.508) (layer F.Cu) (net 10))
 (segment (start 57.2152 28.2572) (end 61.45784 28.2572) (width 0.508) (layer F.Cu) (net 10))
 (segment (start 61.45784 28.2572) (end 65.2152 28.2572) (width 0.508) (layer F.Cu) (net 10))
 (segment (start 65.2152 108.2572) (end 60.97256 108.2572) (width 0.508) (layer B.Cu) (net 9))
 (segment (start 60.97256 108.2572) (end 57.2152 108.2572) (width 0.508) (layer B.Cu) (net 9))
 (segment (start 86.6852 36.0172) (end 71.7804 36.0172) (width 0.508) (layer B.Cu) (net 9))
 (segment (start 71.7804 36.0172) (end 65.2152 42.5824) (width 0.508) (layer B.Cu) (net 9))
 (segment (start 65.2152 42.5824) (end 65.2152 108.2572) (width 0.508) (layer B.Cu) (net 9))
 (segment (start 86.6852 36.0172) (end 86.6852 30.7872) (width 0.508) (layer B.Cu) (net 9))
 (segment (start 86.6852 37.9722) (end 86.6852 36.0172) (width 0.508) (layer B.Cu) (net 9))
 (segment (start 86.6852 30.7872) (end 89.2152 28.2572) (width 0.508) (layer B.Cu) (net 9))
 (segment (start 81.2152 28.2572) (end 85.45784 28.2572) (width 0.508) (layer B.Cu) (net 9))
 (segment (start 85.45784 28.2572) (end 89.2152 28.2572) (width 0.508) (layer B.Cu) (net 9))
 (segment (start 97.2142 28.2572) (end 92.97156 28.2572) (width 0.508) (layer B.Cu) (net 9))
 (segment (start 92.97156 28.2572) (end 89.2152 28.2572) (width 0.508) (layer B.Cu) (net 9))
 (segment (start 84.7852 41.7322) (end 84.7852 44.2722) (width 0.508) (layer F.Cu) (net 9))
 (segment (start 86.6852 39.4512) (end 86.6852 37.9722) (width 0.508) (layer F.Cu) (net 9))
 (segment (start 86.6852 43.0522) (end 86.6852 39.4512) (width 0.508) (layer F.Cu) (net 9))
 (segment (start 84.7852 44.2722) (end 85.4652 44.2722) (width 0.508) (layer F.Cu) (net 9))
 (segment (start 85.4652 44.2722) (end 86.6852 43.0522) (width 0.508) (layer F.Cu) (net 9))
 (segment (start 84.7852 41.7322) (end 84.7852 39.1922) (width 0.508) (layer F.Cu) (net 9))
 (segment (start 84.7852 41.7322) (end 85.4652 41.7322) (width 0.508) (layer F.Cu) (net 9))
 (segment (start 85.4652 41.7322) (end 86.6852 40.5122) (width 0.508) (layer F.Cu) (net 9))
 (segment (start 86.6852 40.5122) (end 86.1052 40.5122) (width 0.508) (layer F.Cu) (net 9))
 (segment (start 86.1052 40.5122) (end 84.7852 39.1922) (width 0.508) (layer F.Cu) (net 9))
 (segment (start 84.7852 39.1922) (end 85.4652 39.1922) (width 0.508) (layer F.Cu) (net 9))
 (segment (start 85.4652 39.1922) (end 86.6852 37.9722) (width 0.508) (layer F.Cu) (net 9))
 (segment (start 57.2152 76.2572) (end 69.8072 88.8492) (width 0.254) (layer F.Cu) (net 14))
 (segment (start 84.7852 87.5522) (end 83.642199 88.695201) (width 0.254) (layer F.Cu) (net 14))
 (segment (start 83.642199 88.695201) (end 83.642199 88.696801) (width 0.254) (layer F.Cu) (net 14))
 (segment (start 83.642199 88.696801) (end 83.4898 88.8492) (width 0.254) (layer F.Cu) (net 14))
 (segment (start 83.4898 88.8492) (end 69.8072 88.8492) (width 0.254) (layer F.Cu) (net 14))
 (segment (start 84.582 102.489) (end 78.9834 102.489) (width 0.254) (layer F.Cu) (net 11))
 (segment (start 78.9834 102.489) (end 73.2152 108.2572) (width 0.254) (layer F.Cu) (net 11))
 (segment (start 88.3158 98.7552) (end 84.582 102.489) (width 0.254) (layer F.Cu) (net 11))
 (segment (start 88.3158 81.026) (end 88.3158 98.7552) (width 0.254) (layer F.Cu) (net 11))
 (segment (start 87.298999 80.009199) (end 88.3158 81.026) (width 0.254) (layer F.Cu) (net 11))
 (segment (start 84.7852 79.9322) (end 85.86283 79.9322) (width 0.254) (layer F.Cu) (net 11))
 (segment (start 85.86283 79.9322) (end 85.939829 80.009199) (width 0.254) (layer F.Cu) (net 11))
 (segment (start 85.939829 80.009199) (end 87.298999 80.009199) (width 0.254) (layer F.Cu) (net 11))
 (segment (start 81.2292 73.542658) (end 79.8322 73.542658) (width 0.1524) (layer F.Cu) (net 17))
 (segment (start 79.8322 73.542658) (end 79.568542 73.542658) (width 0.1524) (layer F.Cu) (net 17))
 (segment (start 57.2152 52.2572) (end 78.500658 73.542658) (width 0.254) (layer F.Cu) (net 17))
 (segment (start 78.500658 73.542658) (end 79.8322 73.542658) (width 0.254) (layer F.Cu) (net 17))
 (segment (start 82.514942 74.8284) (end 81.2292 73.542658) (width 0.1524) (layer F.Cu) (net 17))
 (segment (start 84.7852 77.3922) (end 84.023201 76.630201) (width 0.1524) (layer F.Cu) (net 17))
 (segment (start 84.023201 76.630201) (end 84.023201 75.643743) (width 0.1524) (layer F.Cu) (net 17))
 (segment (start 83.207858 74.8284) (end 82.514942 74.8284) (width 0.1524) (layer F.Cu) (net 17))
 (segment (start 84.023201 75.643743) (end 83.207858 74.8284) (width 0.1524) (layer F.Cu) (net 17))
 (segment (start 81.509457 68.679999) (end 79.629 68.679999) (width 0.1524) (layer F.Cu) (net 18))
 (segment (start 79.629 68.679999) (end 79.503601 68.679999) (width 0.1524) (layer F.Cu) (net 18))
 (segment (start 57.2152 44.2572) (end 60.215199 47.257199) (width 0.254) (layer F.Cu) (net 18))
 (segment (start 60.215199 47.257199) (end 60.215199 49.266198) (width 0.254) (layer F.Cu) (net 18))
 (segment (start 60.215199 49.266198) (end 79.629 68.679999) (width 0.254) (layer F.Cu) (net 18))
 (segment (start 84.7852 69.7722) (end 82.601658 69.7722) (width 0.1524) (layer F.Cu) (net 18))
 (segment (start 82.601658 69.7722) (end 81.509457 68.679999) (width 0.1524) (layer F.Cu) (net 18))
 (segment (start 88.03512 73.688187) (end 88.03512 68.01992) (width 0.254) (layer B.Cu) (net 21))
 (segment (start 88.03512 68.01992) (end 87.2474 67.2322) (width 0.254) (layer B.Cu) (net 21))
 (segment (start 87.2474 67.2322) (end 85.86283 67.2322) (width 0.254) (layer B.Cu) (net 21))
 (segment (start 85.86283 67.2322) (end 84.7852 67.2322) (width 0.254) (layer B.Cu) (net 21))
 (segment (start 88.8746 74.549) (end 88.03512 73.70952) (width 0.254) (layer F.Cu) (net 21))
 (via (at 88.03512 73.688187) (size 0.6858) (drill 0.3302) (layers F.Cu B.Cu) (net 21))
 (segment (start 88.03512 73.70952) (end 88.03512 73.688187) (width 0.254) (layer F.Cu) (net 21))
 (segment (start 81.2152 108.2572) (end 88.8746 100.5978) (width 0.254) (layer F.Cu) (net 21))
 (segment (start 88.8746 100.5978) (end 88.8746 74.549) (width 0.254) (layer F.Cu) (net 21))
 (segment (start 84.7852 59.5122) (end 87.056842 59.5122) (width 0.254) (layer F.Cu) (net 4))
 (segment (start 87.056842 59.5122) (end 93.834199 66.289557) (width 0.254) (layer F.Cu) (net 4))
 (segment (start 93.834199 66.289557) (end 93.834199 72.877199) (width 0.254) (layer F.Cu) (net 4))
 (segment (start 93.834199 72.877199) (end 94.214201 73.257201) (width 0.254) (layer F.Cu) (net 4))
 (segment (start 94.214201 73.257201) (end 97.2142 76.2572) (width 0.254) (layer F.Cu) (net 4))
 (segment (start 84.7852 56.9722) (end 93.9292 56.9722) (width 0.254) (layer F.Cu) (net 2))
 (segment (start 93.9292 56.9722) (end 97.2142 60.2572) (width 0.254) (layer F.Cu) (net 2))
 (segment (start 84.7852 46.8122) (end 94.6592 46.8122) (width 0.254) (layer F.Cu) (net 3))
 (segment (start 94.6592 46.8122) (end 97.2142 44.2572) (width 0.254) (layer F.Cu) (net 3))
 (segment (start 81.509457 81.024401) (end 79.7306 81.024401) (width 0.1524) (layer F.Cu) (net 15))
 (segment (start 79.7306 81.024401) (end 79.170201 81.024401) (width 0.1524) (layer F.Cu) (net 15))
 (segment (start 57.2152 68.2572) (end 69.982401 81.024401) (width 0.254) (layer F.Cu) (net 15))
 (segment (start 69.982401 81.024401) (end 79.7306 81.024401) (width 0.254) (layer F.Cu) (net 15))
 (segment (start 79.170201 81.024401) (end 79.0702 80.9244) (width 0.1524) (layer F.Cu) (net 15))
 (segment (start 86.6852 81.1522) (end 84.451658 81.1522) (width 0.1524) (layer F.Cu) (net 15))
 (segment (start 84.451658 81.1522) (end 83.409457 80.109999) (width 0.1524) (layer F.Cu) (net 15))
 (segment (start 83.409457 80.109999) (end 82.423859 80.109999) (width 0.1524) (layer F.Cu) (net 15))
 (segment (start 82.423859 80.109999) (end 81.509457 81.024401) (width 0.1524) (layer F.Cu) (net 15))
 (segment (start 80.137 75.944401) (end 79.906801 75.944401) (width 0.1524) (layer F.Cu) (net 16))
 (segment (start 81.153859 75.944401) (end 80.137 75.944401) (width 0.1524) (layer F.Cu) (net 16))
 (segment (start 57.2152 60.2572) (end 71.9642 75.0062) (width 0.254) (layer F.Cu) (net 16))
 (segment (start 71.9642 75.0062) (end 72.3706 75.4126) (width 0.254) (layer F.Cu) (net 16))
 (segment (start 80.137 75.944401) (end 72.902401 75.944401) (width 0.254) (layer F.Cu) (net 16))
 (segment (start 72.902401 75.944401) (end 71.9642 75.0062) (width 0.254) (layer F.Cu) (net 16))
 (segment (start 86.6852 78.6122) (end 84.451658 78.6122) (width 0.1524) (layer F.Cu) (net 16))
 (segment (start 84.451658 78.6122) (end 83.157058 77.3176) (width 0.1524) (layer F.Cu) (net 16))
 (segment (start 83.157058 77.3176) (end 82.527058 77.3176) (width 0.1524) (layer F.Cu) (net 16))
 (segment (start 82.527058 77.3176) (end 81.153859 75.944401) (width 0.1524) (layer F.Cu) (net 16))
 (segment (start 90.1192 74.4262) (end 90.1192 85.1612) (width 0.254) (layer F.Cu) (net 8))
 (segment (start 90.1192 85.1612) (end 97.2152 92.2572) (width 0.254) (layer F.Cu) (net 8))
 (segment (start 86.6852 70.9922) (end 90.1192 74.4262) (width 0.254) (layer F.Cu) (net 8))
 (segment (start 78.6384 65.9892) (end 78.6384 57.6804) (width 0.254) (layer F.Cu) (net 19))
 (segment (start 78.6384 57.6804) (end 57.2152 36.2572) (width 0.254) (layer F.Cu) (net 19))
 (segment (start 79.9592 65.9892) (end 79.6798 65.9892) (width 0.1524) (layer F.Cu) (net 19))
 (segment (start 81.358658 65.9892) (end 79.9592 65.9892) (width 0.1524) (layer F.Cu) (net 19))
 (segment (start 79.9592 65.9892) (end 78.6384 65.9892) (width 0.254) (layer F.Cu) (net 19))
 (segment (start 86.6852 68.4522) (end 84.451658 68.4522) (width 0.1524) (layer F.Cu) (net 19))
 (segment (start 84.451658 68.4522) (end 83.053859 67.054401) (width 0.1524) (layer F.Cu) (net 19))
 (segment (start 83.053859 67.054401) (end 82.423859 67.054401) (width 0.1524) (layer F.Cu) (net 19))
 (segment (start 82.423859 67.054401) (end 81.358658 65.9892) (width 0.1524) (layer F.Cu) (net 19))
 (segment (start 86.6852 65.9122) (end 90.932 70.159) (width 0.254) (layer F.Cu) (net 7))
 (segment (start 90.932 77.974) (end 94.215201 81.257201) (width 0.254) (layer F.Cu) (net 7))
 (segment (start 90.932 70.159) (end 90.932 77.974) (width 0.254) (layer F.Cu) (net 7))
 (segment (start 94.215201 81.257201) (end 97.2152 84.2572) (width 0.254) (layer F.Cu) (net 7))
 (segment (start 86.6852 58.2922) (end 96.6502 68.2572) (width 0.254) (layer F.Cu) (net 1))
 (segment (start 96.6502 68.2572) (end 97.2152 68.2572) (width 0.254) (layer F.Cu) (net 1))
 (segment (start 86.6852 55.7522) (end 93.7192 55.7522) (width 0.254) (layer F.Cu) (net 6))
 (segment (start 93.7192 55.7522) (end 97.2142 52.2572) (width 0.254) (layer F.Cu) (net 6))
 (segment (start 86.6852 45.5922) (end 87.8792 45.5922) (width 0.254) (layer F.Cu) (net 5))
 (segment (start 87.8792 45.5922) (end 97.2142 36.2572) (width 0.254) (layer F.Cu) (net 5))
 (segment (start 83.185 91.5162) (end 65.9562 91.5162) (width 0.254) (layer F.Cu) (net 20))
 (segment (start 65.9562 91.5162) (end 57.2152 100.2572) (width 0.254) (layer F.Cu) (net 20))
 (segment (start 86.6852 88.016) (end 83.185 91.5162) (width 0.254) (layer F.Cu) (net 20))
 (segment (start 86.6852 86.2322) (end 86.6852 88.016) (width 0.254) (layer F.Cu) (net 20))
 (segment (start 84.7852 85.0122) (end 85.3652 85.0122) (width 0.254) (layer F.Cu) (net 20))
 (segment (start 85.3652 85.0122) (end 86.6852 83.6922) (width 0.254) (layer F.Cu) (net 20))
 (segment (start 86.6852 83.6922) (end 86.0052 83.6922) (width 0.254) (layer F.Cu) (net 20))
 (segment (start 86.0052 83.6922) (end 84.7852 82.4722) (width 0.254) (layer F.Cu) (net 20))
 (segment (start 86.6852 83.6922) (end 86.6852 84.76983) (width 0.254) (layer F.Cu) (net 20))
 (segment (start 86.6852 84.76983) (end 86.6852 86.2322) (width 0.254) (layer F.Cu) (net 20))
 (segment (start 86.6852 86.2322) (end 86.0052 86.2322) (width 0.254) (layer F.Cu) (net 20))
 (segment (start 86.0052 86.2322) (end 84.7852 85.0122) (width 0.254) (layer F.Cu) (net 20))
 (segment (start 84.7852 82.4722) (end 84.7852 83.54983) (width 0.254) (layer F.Cu) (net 20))
 (segment (start 84.7852 83.54983) (end 84.7852 85.0122) (width 0.254) (layer F.Cu) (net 20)))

